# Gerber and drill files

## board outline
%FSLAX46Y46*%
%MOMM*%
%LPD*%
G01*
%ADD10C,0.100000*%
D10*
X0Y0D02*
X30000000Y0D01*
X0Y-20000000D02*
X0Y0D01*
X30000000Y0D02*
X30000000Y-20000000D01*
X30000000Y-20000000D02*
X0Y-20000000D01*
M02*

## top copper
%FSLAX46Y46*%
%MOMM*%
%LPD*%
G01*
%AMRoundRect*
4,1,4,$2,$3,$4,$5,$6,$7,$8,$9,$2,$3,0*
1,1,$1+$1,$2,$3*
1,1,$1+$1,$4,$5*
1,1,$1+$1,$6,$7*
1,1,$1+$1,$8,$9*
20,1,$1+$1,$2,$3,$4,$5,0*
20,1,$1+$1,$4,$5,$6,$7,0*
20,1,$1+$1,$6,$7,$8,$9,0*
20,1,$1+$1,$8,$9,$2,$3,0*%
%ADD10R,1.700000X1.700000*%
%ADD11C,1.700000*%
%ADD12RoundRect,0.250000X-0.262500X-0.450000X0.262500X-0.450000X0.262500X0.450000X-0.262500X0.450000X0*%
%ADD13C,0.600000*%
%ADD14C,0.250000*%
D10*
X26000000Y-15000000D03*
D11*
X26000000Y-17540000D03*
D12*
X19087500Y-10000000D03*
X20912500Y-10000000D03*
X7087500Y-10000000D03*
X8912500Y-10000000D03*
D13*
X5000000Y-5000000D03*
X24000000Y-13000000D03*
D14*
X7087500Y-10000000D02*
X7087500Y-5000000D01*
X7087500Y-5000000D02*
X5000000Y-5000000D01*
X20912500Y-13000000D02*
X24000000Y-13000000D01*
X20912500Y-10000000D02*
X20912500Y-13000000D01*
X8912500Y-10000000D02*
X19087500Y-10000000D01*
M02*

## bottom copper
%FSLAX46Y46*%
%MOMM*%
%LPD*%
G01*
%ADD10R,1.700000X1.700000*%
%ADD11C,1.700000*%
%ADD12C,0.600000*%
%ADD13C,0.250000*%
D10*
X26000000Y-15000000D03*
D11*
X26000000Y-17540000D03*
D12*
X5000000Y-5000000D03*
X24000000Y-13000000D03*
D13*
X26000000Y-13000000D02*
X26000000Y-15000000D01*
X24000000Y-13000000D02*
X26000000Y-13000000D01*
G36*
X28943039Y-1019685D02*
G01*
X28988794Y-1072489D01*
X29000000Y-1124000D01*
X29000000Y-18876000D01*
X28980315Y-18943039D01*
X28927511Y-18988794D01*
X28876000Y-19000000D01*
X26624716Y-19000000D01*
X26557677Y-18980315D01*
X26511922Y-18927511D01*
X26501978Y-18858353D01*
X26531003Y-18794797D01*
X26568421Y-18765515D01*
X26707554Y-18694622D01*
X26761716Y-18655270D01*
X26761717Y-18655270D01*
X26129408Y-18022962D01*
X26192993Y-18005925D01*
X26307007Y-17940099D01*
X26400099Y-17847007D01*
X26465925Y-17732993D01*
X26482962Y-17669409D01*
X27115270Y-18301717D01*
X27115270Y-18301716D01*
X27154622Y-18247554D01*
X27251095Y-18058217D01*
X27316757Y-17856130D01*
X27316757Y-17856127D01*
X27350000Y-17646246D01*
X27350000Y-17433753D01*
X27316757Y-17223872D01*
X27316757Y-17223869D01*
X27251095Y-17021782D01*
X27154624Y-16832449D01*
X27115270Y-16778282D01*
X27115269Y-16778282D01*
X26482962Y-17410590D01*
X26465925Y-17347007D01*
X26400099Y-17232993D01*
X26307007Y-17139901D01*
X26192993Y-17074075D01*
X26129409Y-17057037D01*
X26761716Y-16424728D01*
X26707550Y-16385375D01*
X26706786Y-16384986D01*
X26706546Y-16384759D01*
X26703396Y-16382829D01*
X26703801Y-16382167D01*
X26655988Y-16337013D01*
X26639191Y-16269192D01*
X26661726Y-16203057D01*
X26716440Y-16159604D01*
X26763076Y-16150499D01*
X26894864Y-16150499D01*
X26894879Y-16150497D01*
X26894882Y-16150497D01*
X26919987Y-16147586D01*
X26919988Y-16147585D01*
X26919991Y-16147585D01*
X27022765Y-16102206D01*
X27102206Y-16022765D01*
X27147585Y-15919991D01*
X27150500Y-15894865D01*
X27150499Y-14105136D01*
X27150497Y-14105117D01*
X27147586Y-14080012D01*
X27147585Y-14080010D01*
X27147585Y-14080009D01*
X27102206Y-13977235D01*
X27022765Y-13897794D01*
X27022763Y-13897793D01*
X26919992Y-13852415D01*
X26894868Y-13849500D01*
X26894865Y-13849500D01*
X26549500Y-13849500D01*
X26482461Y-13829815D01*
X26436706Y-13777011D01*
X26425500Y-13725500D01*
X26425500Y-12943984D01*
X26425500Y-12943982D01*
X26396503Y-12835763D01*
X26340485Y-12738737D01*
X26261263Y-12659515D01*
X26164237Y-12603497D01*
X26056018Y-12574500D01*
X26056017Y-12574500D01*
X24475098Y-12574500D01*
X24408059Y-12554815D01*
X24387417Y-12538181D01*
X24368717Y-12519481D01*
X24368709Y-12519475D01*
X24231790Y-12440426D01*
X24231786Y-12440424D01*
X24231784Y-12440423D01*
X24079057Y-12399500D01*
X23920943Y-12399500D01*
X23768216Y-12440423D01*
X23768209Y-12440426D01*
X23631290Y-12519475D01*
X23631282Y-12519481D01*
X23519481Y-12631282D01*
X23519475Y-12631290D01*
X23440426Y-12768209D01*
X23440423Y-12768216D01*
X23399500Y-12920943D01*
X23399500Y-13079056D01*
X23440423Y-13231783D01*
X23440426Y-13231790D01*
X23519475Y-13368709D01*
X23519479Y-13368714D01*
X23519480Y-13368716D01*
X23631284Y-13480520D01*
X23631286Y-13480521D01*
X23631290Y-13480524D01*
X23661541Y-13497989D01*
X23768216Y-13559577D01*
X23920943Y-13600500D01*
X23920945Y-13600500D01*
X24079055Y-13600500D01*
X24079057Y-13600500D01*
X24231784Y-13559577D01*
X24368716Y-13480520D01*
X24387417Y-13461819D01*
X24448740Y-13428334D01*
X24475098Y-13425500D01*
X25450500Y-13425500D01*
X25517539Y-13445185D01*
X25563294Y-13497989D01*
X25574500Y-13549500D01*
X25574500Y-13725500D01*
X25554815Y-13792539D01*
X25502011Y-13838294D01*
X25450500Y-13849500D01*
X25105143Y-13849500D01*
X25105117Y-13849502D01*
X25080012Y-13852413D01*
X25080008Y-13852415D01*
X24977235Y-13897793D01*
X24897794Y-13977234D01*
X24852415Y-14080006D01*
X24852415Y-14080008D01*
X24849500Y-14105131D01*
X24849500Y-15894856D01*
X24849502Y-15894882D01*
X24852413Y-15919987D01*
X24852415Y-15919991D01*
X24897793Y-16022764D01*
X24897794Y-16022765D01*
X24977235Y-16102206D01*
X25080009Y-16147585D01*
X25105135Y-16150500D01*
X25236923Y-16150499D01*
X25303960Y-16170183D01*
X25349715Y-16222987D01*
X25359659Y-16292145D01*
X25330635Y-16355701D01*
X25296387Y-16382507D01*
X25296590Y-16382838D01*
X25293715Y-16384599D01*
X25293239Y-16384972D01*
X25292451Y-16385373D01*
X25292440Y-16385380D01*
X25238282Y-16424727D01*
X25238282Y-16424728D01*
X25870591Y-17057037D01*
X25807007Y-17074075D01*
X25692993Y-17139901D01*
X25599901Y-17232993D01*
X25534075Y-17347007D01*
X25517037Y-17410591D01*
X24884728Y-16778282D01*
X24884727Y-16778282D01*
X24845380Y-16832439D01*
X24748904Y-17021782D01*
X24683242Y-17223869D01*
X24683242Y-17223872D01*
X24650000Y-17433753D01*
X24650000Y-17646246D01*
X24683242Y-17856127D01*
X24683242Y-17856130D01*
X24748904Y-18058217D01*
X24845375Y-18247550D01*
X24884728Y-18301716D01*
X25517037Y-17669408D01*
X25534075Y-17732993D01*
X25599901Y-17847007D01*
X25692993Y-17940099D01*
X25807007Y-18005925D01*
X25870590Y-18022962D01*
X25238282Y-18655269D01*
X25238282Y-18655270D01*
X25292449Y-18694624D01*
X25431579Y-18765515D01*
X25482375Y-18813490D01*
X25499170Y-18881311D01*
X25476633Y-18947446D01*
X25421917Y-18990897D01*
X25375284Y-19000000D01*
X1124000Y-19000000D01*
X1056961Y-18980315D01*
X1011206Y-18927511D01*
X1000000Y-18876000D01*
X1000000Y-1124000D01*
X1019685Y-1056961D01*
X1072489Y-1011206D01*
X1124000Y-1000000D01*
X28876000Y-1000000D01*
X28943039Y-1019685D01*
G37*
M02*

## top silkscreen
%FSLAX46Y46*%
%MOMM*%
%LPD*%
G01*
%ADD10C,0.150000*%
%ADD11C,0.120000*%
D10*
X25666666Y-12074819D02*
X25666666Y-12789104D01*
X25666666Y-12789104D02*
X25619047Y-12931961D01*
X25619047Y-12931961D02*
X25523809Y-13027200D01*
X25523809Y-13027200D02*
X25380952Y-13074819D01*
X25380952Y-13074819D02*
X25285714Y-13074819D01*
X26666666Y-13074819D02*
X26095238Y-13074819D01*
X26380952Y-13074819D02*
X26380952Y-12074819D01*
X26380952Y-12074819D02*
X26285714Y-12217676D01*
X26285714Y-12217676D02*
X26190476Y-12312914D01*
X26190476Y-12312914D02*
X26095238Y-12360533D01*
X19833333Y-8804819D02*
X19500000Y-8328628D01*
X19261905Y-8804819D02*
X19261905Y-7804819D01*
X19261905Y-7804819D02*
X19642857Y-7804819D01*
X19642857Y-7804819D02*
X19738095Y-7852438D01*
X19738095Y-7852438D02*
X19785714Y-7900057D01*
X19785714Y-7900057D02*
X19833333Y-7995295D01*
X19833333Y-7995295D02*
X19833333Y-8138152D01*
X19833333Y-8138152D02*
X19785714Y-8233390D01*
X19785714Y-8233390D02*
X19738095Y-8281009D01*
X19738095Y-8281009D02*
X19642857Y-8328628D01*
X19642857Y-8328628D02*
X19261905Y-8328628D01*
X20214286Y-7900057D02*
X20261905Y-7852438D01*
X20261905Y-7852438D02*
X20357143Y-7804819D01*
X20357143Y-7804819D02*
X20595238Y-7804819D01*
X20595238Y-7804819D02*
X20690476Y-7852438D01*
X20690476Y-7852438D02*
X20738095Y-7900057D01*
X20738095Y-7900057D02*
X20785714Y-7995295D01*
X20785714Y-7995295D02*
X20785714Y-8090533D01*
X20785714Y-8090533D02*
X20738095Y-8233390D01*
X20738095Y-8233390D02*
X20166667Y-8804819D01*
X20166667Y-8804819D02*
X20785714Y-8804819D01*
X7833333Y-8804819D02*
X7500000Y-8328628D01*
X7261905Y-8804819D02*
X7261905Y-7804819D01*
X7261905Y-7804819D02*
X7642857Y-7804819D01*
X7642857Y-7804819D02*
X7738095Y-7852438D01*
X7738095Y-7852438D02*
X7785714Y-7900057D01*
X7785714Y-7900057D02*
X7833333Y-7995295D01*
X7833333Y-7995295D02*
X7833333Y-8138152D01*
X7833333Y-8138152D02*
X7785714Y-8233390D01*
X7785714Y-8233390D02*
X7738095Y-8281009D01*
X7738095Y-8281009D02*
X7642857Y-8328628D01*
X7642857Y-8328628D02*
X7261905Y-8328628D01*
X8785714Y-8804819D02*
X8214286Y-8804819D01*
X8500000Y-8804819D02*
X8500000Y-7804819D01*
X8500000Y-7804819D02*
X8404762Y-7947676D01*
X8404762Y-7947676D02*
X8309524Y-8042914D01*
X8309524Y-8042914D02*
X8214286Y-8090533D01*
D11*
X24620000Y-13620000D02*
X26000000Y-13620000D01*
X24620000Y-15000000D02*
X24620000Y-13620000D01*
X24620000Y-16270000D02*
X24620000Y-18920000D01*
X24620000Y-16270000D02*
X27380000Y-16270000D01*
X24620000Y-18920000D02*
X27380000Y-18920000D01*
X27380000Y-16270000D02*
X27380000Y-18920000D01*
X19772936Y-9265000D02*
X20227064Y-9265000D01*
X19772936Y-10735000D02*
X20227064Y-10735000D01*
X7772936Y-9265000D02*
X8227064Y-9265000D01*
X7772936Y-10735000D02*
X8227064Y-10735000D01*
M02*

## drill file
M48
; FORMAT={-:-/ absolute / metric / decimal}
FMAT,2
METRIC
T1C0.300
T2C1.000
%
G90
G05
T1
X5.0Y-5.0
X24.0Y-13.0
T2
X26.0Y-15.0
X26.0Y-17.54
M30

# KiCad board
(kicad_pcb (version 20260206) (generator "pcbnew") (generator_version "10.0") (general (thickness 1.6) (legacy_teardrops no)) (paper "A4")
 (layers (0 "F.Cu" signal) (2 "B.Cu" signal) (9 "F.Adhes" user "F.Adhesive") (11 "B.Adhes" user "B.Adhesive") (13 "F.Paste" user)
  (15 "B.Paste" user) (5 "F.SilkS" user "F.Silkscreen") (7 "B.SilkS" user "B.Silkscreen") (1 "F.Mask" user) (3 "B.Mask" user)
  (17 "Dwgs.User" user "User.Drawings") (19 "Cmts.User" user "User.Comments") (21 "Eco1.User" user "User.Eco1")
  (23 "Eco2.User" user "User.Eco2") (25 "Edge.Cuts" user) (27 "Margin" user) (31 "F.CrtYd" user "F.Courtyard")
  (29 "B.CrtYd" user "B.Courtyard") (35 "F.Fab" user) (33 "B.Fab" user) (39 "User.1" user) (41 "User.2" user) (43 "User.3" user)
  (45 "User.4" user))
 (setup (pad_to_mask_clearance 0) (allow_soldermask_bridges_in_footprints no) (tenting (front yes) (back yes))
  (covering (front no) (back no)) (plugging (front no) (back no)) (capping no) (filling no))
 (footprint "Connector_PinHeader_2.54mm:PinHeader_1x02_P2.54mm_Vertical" (layer "F.Cu") (at 26 15)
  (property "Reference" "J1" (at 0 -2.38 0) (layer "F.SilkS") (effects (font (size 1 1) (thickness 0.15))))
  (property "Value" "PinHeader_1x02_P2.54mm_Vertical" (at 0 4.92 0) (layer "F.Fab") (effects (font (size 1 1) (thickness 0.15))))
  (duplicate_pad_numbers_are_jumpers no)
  (fp_line (start -1.38 -1.38) (end 0 -1.38) (stroke (width 0.12) (type solid)) (layer "F.SilkS"))
  (fp_line (start -1.38 0) (end -1.38 -1.38) (stroke (width 0.12) (type solid)) (layer "F.SilkS"))
  (fp_line (start -1.38 1.27) (end -1.38 3.92) (stroke (width 0.12) (type solid)) (layer "F.SilkS"))
  (fp_line (start -1.38 1.27) (end 1.38 1.27) (stroke (width 0.12) (type solid)) (layer "F.SilkS"))
  (fp_line (start -1.38 3.92) (end 1.38 3.92) (stroke (width 0.12) (type solid)) (layer "F.SilkS"))
  (fp_line (start 1.38 1.27) (end 1.38 3.92) (stroke (width 0.12) (type solid)) (layer "F.SilkS"))
  (pad "1" thru_hole rect (at 0 0) (size 1.7 1.7) (drill 1) (layers "*.Cu" "*.Mask") (remove_unused_layers no) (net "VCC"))
  (pad "2" thru_hole circle (at 0 2.54) (size 1.7 1.7) (drill 1) (layers "*.Cu" "*.Mask") (remove_unused_layers no) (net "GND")))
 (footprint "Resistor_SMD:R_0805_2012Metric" (layer "F.Cu") (at 20 10)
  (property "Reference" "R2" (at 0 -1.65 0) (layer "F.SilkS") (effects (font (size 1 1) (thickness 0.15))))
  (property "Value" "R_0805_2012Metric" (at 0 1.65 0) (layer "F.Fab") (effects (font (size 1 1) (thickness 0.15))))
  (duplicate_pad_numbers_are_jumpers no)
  (fp_line (start -0.227064 -0.735) (end 0.227064 -0.735) (stroke (width 0.12) (type solid)) (layer "F.SilkS"))
  (fp_line (start -0.227064 0.735) (end 0.227064 0.735) (stroke (width 0.12) (type solid)) (layer "F.SilkS"))
  (pad "1" smd roundrect (at -0.9125 0) (size 1.025 1.4) (layers "F.Cu" "F.Mask" "F.Paste") (roundrect_rratio 0.243902) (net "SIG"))
  (pad "2" smd roundrect (at 0.9125 0) (size 1.025 1.4) (layers "F.Cu" "F.Mask" "F.Paste") (roundrect_rratio 0.243902) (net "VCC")))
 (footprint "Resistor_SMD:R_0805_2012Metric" (layer "F.Cu") (at 8 10)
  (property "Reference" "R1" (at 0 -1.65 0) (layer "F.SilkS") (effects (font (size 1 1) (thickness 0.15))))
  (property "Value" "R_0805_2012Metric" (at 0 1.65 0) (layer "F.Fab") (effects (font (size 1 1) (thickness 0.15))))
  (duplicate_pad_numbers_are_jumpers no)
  (fp_line (start -0.227064 -0.735) (end 0.227064 -0.735) (stroke (width 0.12) (type solid)) (layer "F.SilkS"))
  (fp_line (start -0.227064 0.735) (end 0.227064 0.735) (stroke (width 0.12) (type solid)) (layer "F.SilkS"))
  (pad "1" smd roundrect (at -0.9125 0) (size 1.025 1.4) (layers "F.Cu" "F.Mask" "F.Paste") (roundrect_rratio 0.243902) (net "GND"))
  (pad "2" smd roundrect (at 0.9125 0) (size 1.025 1.4) (layers "F.Cu" "F.Mask" "F.Paste") (roundrect_rratio 0.243902) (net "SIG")))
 (gr_line (start 0 0) (end 30 0) (stroke (width 0.1) (type default)) (layer "Edge.Cuts"))
 (gr_line (start 0 20) (end 0 0) (stroke (width 0.1) (type default)) (layer "Edge.Cuts"))
 (gr_line (start 30 0) (end 30 20) (stroke (width 0.1) (type default)) (layer "Edge.Cuts"))
 (gr_line (start 30 20) (end 0 20) (stroke (width 0.1) (type default)) (layer "Edge.Cuts"))
 (segment (start 7.0875 10) (end 7.0875 5) (width 0.25) (layer "F.Cu") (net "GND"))
 (segment (start 7.0875 5) (end 5 5) (width 0.25) (layer "F.Cu") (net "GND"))
 (via (at 5 5) (size 0.6) (drill 0.3) (layers "F.Cu" "B.Cu") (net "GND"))
 (segment (start 20.9125 13) (end 24 13) (width 0.25) (layer "F.Cu") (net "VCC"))
 (segment (start 20.9125 10) (end 20.9125 13) (width 0.25) (layer "F.Cu") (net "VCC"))
 (via (at 24 13) (size 0.6) (drill 0.3) (layers "F.Cu" "B.Cu") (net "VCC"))
 (segment (start 26 13) (end 26 15) (width 0.25) (layer "B.Cu") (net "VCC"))
 (segment (start 24 13) (end 26 13) (width 0.25) (layer "B.Cu") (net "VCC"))
 (segment (start 8.9125 10) (end 19.0875 10) (width 0.25) (layer "F.Cu") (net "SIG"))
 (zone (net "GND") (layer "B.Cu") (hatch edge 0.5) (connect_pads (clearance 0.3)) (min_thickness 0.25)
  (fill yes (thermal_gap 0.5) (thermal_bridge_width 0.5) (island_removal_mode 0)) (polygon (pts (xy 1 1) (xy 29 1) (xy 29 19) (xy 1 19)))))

